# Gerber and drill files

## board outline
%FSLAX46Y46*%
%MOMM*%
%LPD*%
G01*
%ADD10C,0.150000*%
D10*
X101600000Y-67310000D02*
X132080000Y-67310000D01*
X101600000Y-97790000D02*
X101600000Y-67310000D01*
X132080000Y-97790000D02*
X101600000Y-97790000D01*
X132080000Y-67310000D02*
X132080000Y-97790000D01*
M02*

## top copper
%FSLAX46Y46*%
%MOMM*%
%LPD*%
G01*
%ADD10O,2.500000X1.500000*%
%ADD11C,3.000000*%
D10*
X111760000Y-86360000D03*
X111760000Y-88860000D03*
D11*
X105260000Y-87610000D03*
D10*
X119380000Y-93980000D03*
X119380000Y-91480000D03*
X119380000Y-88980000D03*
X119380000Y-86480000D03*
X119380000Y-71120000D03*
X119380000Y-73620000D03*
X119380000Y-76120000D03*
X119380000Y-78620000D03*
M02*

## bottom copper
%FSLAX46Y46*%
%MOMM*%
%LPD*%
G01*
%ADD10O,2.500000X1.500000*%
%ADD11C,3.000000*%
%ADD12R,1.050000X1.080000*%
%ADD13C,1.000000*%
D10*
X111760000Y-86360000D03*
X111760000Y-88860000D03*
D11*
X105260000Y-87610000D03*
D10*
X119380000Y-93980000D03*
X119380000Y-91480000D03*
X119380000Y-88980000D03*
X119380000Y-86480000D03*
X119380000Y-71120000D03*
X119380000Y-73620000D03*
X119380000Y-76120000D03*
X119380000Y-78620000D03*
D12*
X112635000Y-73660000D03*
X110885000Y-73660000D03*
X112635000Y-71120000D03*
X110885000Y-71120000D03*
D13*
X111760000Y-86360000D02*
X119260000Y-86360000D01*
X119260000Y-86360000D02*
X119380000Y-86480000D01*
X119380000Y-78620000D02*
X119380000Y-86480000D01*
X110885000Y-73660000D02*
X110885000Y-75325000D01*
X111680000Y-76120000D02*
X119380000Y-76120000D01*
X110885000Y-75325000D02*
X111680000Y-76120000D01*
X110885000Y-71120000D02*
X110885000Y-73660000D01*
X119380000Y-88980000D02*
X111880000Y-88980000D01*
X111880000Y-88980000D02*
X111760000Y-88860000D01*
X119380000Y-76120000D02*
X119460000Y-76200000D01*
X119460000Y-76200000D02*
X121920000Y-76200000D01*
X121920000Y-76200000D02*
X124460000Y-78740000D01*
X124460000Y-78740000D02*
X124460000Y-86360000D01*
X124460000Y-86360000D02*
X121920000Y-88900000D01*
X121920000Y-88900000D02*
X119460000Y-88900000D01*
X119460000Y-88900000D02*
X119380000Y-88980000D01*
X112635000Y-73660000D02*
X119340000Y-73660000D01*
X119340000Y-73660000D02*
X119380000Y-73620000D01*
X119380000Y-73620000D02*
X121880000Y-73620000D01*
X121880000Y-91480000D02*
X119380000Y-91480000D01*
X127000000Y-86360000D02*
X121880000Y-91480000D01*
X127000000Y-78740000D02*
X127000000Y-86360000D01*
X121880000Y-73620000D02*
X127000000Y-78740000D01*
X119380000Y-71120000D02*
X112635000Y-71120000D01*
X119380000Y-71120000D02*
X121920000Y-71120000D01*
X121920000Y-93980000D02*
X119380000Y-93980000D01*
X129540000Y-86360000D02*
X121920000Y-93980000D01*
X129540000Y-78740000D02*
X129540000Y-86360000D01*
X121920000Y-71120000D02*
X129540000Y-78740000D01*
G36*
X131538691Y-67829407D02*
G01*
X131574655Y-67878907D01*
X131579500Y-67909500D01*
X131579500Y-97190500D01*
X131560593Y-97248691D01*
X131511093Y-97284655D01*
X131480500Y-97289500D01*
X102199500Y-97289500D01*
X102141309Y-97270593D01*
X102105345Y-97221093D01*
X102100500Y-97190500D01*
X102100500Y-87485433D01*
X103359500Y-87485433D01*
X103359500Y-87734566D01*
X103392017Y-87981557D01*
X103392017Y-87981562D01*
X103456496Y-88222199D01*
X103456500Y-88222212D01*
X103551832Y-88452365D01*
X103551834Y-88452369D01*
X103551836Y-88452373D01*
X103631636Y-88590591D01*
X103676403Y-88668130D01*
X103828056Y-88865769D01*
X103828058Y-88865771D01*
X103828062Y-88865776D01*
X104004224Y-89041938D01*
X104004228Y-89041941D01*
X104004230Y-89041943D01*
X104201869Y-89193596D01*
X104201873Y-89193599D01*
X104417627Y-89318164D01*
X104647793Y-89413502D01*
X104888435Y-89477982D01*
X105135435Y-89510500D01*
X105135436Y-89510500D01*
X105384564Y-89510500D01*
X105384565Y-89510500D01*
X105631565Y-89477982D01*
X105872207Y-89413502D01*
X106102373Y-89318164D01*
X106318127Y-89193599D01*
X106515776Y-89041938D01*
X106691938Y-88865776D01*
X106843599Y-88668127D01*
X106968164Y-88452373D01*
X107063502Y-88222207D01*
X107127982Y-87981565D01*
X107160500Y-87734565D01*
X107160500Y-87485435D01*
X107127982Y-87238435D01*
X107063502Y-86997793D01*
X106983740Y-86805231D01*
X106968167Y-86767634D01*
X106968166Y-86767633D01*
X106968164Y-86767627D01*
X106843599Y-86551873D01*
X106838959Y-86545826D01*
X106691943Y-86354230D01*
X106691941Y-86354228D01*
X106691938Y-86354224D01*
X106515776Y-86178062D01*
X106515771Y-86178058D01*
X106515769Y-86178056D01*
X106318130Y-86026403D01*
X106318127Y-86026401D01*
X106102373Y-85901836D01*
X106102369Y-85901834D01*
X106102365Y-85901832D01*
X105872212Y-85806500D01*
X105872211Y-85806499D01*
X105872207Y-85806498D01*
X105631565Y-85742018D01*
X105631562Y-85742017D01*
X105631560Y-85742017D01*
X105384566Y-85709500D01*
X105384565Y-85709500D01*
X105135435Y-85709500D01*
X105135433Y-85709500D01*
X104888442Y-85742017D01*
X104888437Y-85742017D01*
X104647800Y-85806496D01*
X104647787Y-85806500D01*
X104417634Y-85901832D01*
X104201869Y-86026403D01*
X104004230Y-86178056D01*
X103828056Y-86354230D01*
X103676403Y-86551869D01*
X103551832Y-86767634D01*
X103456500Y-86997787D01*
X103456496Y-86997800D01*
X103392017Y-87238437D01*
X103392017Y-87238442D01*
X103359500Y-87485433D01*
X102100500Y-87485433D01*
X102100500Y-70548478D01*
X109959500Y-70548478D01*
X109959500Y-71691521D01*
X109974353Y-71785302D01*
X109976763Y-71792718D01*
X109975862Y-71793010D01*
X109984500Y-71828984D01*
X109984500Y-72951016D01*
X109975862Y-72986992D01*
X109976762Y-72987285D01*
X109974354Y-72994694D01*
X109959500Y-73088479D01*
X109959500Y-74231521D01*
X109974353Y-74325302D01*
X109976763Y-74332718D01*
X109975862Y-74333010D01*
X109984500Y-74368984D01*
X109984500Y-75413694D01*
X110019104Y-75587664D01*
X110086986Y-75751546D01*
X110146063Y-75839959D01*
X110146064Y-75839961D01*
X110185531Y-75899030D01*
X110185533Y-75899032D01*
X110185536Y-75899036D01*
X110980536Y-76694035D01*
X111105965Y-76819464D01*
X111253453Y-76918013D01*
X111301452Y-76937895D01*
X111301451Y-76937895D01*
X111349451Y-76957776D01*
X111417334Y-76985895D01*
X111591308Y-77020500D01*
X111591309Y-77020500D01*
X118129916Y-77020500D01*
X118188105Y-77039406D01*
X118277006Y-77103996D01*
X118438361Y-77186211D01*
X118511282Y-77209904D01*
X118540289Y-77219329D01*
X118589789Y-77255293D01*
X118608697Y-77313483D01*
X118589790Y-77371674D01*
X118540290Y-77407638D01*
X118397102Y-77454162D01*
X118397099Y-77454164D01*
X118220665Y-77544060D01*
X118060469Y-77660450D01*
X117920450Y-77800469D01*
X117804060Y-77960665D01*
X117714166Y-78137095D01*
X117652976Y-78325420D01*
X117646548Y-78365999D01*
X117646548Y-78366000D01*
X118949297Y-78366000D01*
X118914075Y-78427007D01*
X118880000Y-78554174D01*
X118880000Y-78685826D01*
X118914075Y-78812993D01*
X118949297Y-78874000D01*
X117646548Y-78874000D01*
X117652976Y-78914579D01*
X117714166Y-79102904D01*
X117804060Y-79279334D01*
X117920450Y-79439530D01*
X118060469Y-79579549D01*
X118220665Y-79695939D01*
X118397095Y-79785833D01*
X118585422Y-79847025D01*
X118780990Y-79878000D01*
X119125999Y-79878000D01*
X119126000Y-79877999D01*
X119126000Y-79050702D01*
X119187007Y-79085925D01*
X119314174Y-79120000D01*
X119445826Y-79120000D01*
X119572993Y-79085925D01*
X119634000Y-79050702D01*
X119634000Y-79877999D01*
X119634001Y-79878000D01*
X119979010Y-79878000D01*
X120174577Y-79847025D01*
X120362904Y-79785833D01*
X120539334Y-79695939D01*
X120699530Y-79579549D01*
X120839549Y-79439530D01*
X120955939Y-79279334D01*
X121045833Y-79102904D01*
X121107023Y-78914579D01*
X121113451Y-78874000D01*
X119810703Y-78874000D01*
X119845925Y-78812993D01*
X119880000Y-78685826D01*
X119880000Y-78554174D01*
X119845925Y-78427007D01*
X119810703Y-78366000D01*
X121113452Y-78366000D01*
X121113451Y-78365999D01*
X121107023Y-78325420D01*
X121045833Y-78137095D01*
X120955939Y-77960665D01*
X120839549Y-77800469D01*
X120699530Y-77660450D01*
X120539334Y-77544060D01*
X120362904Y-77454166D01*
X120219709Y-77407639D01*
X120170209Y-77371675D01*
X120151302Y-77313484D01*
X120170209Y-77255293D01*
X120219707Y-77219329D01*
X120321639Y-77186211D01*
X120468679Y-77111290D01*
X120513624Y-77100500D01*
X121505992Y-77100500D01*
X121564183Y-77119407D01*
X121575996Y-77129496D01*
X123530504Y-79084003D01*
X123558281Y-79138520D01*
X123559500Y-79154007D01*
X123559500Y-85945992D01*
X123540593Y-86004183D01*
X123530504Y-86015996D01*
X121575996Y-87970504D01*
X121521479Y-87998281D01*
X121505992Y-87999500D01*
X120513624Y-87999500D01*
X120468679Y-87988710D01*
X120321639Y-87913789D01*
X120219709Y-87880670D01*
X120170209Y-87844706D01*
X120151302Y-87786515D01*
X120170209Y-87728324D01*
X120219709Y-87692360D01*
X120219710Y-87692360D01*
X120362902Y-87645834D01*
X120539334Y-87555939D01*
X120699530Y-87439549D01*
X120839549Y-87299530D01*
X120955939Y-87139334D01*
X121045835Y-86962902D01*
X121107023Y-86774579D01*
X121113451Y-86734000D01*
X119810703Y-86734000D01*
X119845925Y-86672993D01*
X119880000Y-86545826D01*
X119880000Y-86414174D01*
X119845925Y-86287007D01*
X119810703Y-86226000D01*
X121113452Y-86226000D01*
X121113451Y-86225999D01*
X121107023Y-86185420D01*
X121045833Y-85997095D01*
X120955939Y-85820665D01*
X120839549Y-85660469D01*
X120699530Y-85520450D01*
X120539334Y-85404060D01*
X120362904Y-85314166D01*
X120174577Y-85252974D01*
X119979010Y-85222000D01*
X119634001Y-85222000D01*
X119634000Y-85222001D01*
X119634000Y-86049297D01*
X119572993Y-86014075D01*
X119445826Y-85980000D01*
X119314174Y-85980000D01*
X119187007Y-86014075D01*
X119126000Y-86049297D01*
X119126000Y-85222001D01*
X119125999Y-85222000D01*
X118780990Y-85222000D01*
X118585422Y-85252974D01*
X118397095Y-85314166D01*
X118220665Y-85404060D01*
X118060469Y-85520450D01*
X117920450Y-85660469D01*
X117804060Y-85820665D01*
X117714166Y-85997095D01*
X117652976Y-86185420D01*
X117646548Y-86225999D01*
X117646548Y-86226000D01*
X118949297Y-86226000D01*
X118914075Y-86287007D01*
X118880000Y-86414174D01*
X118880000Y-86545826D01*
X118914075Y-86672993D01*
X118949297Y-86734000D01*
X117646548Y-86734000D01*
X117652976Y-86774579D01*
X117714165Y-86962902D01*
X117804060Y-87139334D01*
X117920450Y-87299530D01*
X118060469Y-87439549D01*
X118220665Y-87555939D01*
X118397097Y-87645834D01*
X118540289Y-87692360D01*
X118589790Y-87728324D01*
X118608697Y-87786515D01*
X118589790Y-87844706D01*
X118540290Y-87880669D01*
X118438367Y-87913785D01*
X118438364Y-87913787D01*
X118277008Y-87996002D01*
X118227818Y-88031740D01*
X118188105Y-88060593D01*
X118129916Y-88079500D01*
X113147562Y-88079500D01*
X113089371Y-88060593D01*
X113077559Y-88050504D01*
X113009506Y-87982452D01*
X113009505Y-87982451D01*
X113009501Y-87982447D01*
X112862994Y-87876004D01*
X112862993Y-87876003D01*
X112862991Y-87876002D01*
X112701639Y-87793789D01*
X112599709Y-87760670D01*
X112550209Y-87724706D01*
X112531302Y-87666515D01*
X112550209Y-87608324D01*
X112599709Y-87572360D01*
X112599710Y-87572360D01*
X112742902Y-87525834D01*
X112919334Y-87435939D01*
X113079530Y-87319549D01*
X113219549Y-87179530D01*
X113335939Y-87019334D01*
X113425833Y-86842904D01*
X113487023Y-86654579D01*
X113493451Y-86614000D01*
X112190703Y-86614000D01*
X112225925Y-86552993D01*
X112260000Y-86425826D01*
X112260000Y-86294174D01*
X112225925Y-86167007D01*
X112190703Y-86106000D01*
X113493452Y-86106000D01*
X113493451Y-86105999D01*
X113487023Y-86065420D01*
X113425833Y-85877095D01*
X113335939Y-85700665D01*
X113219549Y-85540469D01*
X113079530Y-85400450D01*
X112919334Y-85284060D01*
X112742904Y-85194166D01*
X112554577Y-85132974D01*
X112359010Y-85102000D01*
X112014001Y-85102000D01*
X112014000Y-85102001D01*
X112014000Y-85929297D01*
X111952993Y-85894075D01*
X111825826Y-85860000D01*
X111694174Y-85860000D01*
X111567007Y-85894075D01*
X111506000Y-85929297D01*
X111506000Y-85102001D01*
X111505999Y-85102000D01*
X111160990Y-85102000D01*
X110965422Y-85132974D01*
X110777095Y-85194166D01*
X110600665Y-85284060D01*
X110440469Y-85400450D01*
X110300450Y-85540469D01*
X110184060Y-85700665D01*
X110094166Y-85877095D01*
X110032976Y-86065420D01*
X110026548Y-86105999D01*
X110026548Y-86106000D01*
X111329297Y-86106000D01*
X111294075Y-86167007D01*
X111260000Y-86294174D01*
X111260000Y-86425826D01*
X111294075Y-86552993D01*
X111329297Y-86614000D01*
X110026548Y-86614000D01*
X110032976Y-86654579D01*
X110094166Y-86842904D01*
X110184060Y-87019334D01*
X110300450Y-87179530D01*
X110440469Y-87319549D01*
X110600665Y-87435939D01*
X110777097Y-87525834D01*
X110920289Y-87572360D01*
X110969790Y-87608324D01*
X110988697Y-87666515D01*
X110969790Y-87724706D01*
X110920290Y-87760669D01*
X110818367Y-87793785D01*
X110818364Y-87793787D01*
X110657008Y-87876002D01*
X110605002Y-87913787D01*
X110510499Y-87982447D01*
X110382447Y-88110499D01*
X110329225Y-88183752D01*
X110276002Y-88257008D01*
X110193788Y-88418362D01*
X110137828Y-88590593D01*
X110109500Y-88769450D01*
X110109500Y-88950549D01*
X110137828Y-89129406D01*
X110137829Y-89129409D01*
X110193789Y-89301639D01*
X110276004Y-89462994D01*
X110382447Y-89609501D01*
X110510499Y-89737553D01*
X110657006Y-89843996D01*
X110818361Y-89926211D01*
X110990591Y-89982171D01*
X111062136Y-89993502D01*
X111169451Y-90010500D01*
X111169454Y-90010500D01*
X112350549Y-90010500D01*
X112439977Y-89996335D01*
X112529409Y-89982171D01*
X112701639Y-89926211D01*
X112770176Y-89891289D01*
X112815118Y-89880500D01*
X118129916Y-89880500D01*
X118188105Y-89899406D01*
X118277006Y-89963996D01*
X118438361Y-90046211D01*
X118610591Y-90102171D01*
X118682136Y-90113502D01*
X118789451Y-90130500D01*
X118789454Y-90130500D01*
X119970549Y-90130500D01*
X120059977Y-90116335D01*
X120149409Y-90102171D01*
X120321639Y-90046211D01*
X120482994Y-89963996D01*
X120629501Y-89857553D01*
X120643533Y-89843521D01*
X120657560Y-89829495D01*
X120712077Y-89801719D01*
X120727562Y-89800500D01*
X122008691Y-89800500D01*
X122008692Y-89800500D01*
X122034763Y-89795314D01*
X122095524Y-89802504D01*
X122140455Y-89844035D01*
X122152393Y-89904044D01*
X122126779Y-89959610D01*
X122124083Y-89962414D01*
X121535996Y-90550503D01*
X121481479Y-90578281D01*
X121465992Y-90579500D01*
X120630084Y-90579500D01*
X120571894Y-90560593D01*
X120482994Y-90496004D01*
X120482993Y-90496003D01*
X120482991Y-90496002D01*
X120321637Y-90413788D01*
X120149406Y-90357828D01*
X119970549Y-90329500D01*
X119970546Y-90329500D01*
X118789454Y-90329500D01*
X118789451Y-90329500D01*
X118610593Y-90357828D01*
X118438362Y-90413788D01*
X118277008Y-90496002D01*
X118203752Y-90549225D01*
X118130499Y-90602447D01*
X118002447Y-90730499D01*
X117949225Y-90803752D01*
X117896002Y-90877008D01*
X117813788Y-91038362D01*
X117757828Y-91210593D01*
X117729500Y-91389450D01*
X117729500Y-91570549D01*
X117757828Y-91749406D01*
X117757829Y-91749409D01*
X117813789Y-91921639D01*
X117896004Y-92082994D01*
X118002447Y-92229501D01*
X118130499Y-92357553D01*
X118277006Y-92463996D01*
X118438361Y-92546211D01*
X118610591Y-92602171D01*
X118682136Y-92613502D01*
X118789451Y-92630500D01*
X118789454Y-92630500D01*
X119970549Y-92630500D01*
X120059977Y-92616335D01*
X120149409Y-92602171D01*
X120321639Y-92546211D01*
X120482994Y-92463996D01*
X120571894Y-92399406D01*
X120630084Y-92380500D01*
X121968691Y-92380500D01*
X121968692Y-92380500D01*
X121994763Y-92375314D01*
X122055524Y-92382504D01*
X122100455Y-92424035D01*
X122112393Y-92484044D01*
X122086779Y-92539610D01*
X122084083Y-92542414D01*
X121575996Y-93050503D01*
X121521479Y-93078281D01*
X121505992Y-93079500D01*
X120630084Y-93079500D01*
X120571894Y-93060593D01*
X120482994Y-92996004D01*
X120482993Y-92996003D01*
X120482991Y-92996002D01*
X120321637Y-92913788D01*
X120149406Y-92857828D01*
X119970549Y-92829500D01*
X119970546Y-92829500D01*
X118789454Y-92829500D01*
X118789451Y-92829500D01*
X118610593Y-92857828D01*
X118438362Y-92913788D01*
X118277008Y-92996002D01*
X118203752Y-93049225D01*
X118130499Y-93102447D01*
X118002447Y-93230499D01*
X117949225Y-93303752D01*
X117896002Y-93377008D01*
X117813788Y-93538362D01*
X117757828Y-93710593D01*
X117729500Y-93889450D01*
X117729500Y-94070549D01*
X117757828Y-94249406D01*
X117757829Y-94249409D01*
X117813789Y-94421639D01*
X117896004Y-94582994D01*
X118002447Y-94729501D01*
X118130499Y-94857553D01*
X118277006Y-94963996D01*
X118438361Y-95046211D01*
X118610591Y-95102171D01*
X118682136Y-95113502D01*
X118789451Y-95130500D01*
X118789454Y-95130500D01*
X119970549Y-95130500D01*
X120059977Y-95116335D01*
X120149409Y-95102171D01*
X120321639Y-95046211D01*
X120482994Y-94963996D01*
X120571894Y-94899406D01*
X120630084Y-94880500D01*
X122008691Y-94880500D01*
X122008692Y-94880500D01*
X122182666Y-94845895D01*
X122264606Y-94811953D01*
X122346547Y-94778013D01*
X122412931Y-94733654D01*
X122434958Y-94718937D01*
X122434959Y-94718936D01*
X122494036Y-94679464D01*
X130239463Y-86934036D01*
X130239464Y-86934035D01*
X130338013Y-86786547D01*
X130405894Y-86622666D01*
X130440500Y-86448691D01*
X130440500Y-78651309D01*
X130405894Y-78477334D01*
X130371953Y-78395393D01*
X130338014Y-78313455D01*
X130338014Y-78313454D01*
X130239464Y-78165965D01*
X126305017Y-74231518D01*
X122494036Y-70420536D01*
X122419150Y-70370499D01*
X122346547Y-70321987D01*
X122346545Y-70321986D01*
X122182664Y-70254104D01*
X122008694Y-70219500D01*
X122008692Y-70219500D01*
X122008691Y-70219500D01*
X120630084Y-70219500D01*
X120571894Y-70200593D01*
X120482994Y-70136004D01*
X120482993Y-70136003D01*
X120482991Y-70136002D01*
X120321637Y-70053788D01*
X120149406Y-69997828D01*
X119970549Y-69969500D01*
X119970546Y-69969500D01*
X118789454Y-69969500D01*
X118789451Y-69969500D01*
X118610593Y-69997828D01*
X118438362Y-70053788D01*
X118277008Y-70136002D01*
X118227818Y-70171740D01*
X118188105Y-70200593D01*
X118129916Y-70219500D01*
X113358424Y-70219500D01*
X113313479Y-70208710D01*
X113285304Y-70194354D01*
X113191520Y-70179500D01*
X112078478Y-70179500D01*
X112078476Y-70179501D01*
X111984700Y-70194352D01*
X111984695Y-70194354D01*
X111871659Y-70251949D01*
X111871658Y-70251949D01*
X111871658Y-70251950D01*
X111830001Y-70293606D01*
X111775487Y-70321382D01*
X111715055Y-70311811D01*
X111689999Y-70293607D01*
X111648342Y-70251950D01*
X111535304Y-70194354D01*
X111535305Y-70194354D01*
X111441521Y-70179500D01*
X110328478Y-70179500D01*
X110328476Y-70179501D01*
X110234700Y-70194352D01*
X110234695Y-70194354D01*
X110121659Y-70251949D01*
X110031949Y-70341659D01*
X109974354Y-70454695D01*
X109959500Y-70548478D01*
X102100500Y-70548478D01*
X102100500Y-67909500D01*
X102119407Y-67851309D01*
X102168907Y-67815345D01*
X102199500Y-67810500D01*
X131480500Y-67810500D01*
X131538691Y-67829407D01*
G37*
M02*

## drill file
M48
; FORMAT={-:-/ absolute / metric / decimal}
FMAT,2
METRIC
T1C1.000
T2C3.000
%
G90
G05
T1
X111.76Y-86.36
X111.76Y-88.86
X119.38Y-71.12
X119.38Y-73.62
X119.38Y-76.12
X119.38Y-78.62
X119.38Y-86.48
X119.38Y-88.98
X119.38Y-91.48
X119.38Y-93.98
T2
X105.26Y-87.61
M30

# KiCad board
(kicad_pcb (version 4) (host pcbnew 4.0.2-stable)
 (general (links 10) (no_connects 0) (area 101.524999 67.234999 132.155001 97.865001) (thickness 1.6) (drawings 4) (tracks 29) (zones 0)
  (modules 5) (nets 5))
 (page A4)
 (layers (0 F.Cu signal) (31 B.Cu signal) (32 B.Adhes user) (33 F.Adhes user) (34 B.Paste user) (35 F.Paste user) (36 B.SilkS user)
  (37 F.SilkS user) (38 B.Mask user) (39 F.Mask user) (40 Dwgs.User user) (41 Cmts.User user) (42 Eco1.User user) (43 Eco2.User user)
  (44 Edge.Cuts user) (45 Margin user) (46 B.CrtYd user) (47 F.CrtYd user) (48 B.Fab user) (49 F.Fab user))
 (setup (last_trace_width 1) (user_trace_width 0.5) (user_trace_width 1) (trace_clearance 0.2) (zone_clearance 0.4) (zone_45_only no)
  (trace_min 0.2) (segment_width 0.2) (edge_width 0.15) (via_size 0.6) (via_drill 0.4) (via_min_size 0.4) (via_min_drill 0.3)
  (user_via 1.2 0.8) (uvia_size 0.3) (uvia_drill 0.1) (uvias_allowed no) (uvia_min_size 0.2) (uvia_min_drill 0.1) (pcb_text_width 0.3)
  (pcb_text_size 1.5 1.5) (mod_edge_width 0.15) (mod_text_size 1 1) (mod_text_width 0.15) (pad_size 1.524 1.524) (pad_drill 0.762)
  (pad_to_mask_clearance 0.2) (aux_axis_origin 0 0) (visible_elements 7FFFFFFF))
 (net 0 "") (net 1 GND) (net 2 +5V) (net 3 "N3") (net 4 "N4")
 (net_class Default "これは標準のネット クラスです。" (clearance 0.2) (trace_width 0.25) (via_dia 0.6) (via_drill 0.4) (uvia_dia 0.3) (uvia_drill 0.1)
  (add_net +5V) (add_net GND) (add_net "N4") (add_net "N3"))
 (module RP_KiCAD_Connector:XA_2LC (layer F.Cu) (at 111.76 86.36 270)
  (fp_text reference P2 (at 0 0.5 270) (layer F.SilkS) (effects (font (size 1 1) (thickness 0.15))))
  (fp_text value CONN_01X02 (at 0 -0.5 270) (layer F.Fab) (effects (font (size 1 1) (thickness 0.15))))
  (pad 1 thru_hole oval (at 0 0 270) (size 1.5 2.5) (drill 1) (layers *.Cu *.Mask F.SilkS) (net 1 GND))
  (pad 2 thru_hole oval (at 2.5 0 270) (size 1.5 2.5) (drill 1) (layers *.Cu *.Mask F.SilkS) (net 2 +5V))
  (pad "" thru_hole circle (at 1.25 6.5 270) (size 3 3) (drill 3) (layers *.Cu *.Mask F.SilkS) (clearance -0.3)))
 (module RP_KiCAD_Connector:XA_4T (layer F.Cu) (at 119.38 93.98 90)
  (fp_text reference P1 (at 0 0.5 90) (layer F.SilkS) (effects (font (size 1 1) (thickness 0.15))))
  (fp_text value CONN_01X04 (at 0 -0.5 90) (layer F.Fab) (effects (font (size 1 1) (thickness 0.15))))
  (pad 4 thru_hole oval (at 0 0 90) (size 1.5 2.5) (drill 1) (layers *.Cu *.Mask F.SilkS) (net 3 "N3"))
  (pad 3 thru_hole oval (at 2.5 0 90) (size 1.5 2.5) (drill 1) (layers *.Cu *.Mask F.SilkS) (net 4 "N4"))
  (pad 2 thru_hole oval (at 5 0 90) (size 1.5 2.5) (drill 1) (layers *.Cu *.Mask F.SilkS) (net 2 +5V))
  (pad 1 thru_hole oval (at 7.5 0 90) (size 1.5 2.5) (drill 1) (layers *.Cu *.Mask F.SilkS) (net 1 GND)))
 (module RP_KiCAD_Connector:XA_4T (layer F.Cu) (at 119.38 71.12 270)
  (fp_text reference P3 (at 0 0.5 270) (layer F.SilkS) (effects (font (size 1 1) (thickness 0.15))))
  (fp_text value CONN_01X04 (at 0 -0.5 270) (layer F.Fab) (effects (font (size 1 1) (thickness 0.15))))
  (pad 4 thru_hole oval (at 0 0 270) (size 1.5 2.5) (drill 1) (layers *.Cu *.Mask F.SilkS) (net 3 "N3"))
  (pad 3 thru_hole oval (at 2.5 0 270) (size 1.5 2.5) (drill 1) (layers *.Cu *.Mask F.SilkS) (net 4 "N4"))
  (pad 2 thru_hole oval (at 5 0 270) (size 1.5 2.5) (drill 1) (layers *.Cu *.Mask F.SilkS) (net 2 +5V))
  (pad 1 thru_hole oval (at 7.5 0 270) (size 1.5 2.5) (drill 1) (layers *.Cu *.Mask F.SilkS) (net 1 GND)))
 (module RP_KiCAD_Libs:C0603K (layer B.Cu) (at 111.76 73.66 180)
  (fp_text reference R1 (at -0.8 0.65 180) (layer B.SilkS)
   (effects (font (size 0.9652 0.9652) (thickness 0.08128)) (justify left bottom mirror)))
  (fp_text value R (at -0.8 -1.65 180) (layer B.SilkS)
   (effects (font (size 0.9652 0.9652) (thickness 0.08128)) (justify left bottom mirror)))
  (pad 1 smd rect (at -0.875 0 180) (size 1.05 1.08) (layers B.Cu B.Paste B.Mask) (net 4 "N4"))
  (pad 2 smd rect (at 0.875 0 180) (size 1.05 1.08) (layers B.Cu B.Paste B.Mask) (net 2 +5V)))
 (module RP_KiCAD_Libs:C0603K (layer B.Cu) (at 111.76 71.12 180)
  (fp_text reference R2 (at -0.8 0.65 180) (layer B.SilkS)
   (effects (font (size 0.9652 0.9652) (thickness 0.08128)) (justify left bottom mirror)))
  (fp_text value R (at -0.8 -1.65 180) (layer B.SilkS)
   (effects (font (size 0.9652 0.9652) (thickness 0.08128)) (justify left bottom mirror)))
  (pad 1 smd rect (at -0.875 0 180) (size 1.05 1.08) (layers B.Cu B.Paste B.Mask) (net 3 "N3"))
  (pad 2 smd rect (at 0.875 0 180) (size 1.05 1.08) (layers B.Cu B.Paste B.Mask) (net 2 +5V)))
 (gr_line (start 101.6 67.31) (end 132.08 67.31) (angle 90) (layer Edge.Cuts) (width 0.15))
 (gr_line (start 101.6 97.79) (end 101.6 67.31) (angle 90) (layer Edge.Cuts) (width 0.15))
 (gr_line (start 132.08 97.79) (end 101.6 97.79) (angle 90) (layer Edge.Cuts) (width 0.15))
 (gr_line (start 132.08 67.31) (end 132.08 97.79) (angle 90) (layer Edge.Cuts) (width 0.15))
 (segment (start 111.76 86.36) (end 119.26 86.36) (width 1) (layer B.Cu) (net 1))
 (segment (start 119.26 86.36) (end 119.38 86.48) (width 1) (layer B.Cu) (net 1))
 (segment (start 119.38 78.62) (end 119.38 86.48) (width 1) (layer B.Cu) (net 1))
 (segment (start 110.885 73.66) (end 110.885 75.325) (width 1) (layer B.Cu) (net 2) (status 400000))
 (segment (start 111.68 76.12) (end 119.38 76.12) (width 1) (layer B.Cu) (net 2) (status 800000))
 (segment (start 110.885 75.325) (end 111.68 76.12) (width 1) (layer B.Cu) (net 2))
 (segment (start 110.885 71.12) (end 110.885 73.66) (width 1) (layer B.Cu) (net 2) (status C00000))
 (segment (start 119.38 88.98) (end 111.88 88.98) (width 1) (layer B.Cu) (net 2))
 (segment (start 111.88 88.98) (end 111.76 88.86) (width 1) (layer B.Cu) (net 2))
 (segment (start 119.38 76.12) (end 119.46 76.2) (width 1) (layer B.Cu) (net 2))
 (segment (start 119.46 76.2) (end 121.92 76.2) (width 1) (layer B.Cu) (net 2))
 (segment (start 121.92 76.2) (end 124.46 78.74) (width 1) (layer B.Cu) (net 2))
 (segment (start 124.46 78.74) (end 124.46 86.36) (width 1) (layer B.Cu) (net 2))
 (segment (start 124.46 86.36) (end 121.92 88.9) (width 1) (layer B.Cu) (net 2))
 (segment (start 121.92 88.9) (end 119.46 88.9) (width 1) (layer B.Cu) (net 2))
 (segment (start 119.46 88.9) (end 119.38 88.98) (width 1) (layer B.Cu) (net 2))
 (segment (start 112.635 73.66) (end 119.34 73.66) (width 1) (layer B.Cu) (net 4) (status C00000))
 (segment (start 119.34 73.66) (end 119.38 73.62) (width 1) (layer B.Cu) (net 4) (status C00000))
 (segment (start 119.38 73.62) (end 121.88 73.62) (width 1) (layer B.Cu) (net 4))
 (segment (start 121.88 91.48) (end 119.38 91.48) (width 1) (layer B.Cu) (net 4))
 (segment (start 127 86.36) (end 121.88 91.48) (width 1) (layer B.Cu) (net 4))
 (segment (start 127 78.74) (end 127 86.36) (width 1) (layer B.Cu) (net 4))
 (segment (start 121.88 73.62) (end 127 78.74) (width 1) (layer B.Cu) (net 4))
 (segment (start 119.38 71.12) (end 112.635 71.12) (width 1) (layer B.Cu) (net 3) (status C00000))
 (segment (start 119.38 71.12) (end 121.92 71.12) (width 1) (layer B.Cu) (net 3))
 (segment (start 121.92 93.98) (end 119.38 93.98) (width 1) (layer B.Cu) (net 3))
 (segment (start 129.54 86.36) (end 121.92 93.98) (width 1) (layer B.Cu) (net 3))
 (segment (start 129.54 78.74) (end 129.54 86.36) (width 1) (layer B.Cu) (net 3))
 (segment (start 121.92 71.12) (end 129.54 78.74) (width 1) (layer B.Cu) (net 3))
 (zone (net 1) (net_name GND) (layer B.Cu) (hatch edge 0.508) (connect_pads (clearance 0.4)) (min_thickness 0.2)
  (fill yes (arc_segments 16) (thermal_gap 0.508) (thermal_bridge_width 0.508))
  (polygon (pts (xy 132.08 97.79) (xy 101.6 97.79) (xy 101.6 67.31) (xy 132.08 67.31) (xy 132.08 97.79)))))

